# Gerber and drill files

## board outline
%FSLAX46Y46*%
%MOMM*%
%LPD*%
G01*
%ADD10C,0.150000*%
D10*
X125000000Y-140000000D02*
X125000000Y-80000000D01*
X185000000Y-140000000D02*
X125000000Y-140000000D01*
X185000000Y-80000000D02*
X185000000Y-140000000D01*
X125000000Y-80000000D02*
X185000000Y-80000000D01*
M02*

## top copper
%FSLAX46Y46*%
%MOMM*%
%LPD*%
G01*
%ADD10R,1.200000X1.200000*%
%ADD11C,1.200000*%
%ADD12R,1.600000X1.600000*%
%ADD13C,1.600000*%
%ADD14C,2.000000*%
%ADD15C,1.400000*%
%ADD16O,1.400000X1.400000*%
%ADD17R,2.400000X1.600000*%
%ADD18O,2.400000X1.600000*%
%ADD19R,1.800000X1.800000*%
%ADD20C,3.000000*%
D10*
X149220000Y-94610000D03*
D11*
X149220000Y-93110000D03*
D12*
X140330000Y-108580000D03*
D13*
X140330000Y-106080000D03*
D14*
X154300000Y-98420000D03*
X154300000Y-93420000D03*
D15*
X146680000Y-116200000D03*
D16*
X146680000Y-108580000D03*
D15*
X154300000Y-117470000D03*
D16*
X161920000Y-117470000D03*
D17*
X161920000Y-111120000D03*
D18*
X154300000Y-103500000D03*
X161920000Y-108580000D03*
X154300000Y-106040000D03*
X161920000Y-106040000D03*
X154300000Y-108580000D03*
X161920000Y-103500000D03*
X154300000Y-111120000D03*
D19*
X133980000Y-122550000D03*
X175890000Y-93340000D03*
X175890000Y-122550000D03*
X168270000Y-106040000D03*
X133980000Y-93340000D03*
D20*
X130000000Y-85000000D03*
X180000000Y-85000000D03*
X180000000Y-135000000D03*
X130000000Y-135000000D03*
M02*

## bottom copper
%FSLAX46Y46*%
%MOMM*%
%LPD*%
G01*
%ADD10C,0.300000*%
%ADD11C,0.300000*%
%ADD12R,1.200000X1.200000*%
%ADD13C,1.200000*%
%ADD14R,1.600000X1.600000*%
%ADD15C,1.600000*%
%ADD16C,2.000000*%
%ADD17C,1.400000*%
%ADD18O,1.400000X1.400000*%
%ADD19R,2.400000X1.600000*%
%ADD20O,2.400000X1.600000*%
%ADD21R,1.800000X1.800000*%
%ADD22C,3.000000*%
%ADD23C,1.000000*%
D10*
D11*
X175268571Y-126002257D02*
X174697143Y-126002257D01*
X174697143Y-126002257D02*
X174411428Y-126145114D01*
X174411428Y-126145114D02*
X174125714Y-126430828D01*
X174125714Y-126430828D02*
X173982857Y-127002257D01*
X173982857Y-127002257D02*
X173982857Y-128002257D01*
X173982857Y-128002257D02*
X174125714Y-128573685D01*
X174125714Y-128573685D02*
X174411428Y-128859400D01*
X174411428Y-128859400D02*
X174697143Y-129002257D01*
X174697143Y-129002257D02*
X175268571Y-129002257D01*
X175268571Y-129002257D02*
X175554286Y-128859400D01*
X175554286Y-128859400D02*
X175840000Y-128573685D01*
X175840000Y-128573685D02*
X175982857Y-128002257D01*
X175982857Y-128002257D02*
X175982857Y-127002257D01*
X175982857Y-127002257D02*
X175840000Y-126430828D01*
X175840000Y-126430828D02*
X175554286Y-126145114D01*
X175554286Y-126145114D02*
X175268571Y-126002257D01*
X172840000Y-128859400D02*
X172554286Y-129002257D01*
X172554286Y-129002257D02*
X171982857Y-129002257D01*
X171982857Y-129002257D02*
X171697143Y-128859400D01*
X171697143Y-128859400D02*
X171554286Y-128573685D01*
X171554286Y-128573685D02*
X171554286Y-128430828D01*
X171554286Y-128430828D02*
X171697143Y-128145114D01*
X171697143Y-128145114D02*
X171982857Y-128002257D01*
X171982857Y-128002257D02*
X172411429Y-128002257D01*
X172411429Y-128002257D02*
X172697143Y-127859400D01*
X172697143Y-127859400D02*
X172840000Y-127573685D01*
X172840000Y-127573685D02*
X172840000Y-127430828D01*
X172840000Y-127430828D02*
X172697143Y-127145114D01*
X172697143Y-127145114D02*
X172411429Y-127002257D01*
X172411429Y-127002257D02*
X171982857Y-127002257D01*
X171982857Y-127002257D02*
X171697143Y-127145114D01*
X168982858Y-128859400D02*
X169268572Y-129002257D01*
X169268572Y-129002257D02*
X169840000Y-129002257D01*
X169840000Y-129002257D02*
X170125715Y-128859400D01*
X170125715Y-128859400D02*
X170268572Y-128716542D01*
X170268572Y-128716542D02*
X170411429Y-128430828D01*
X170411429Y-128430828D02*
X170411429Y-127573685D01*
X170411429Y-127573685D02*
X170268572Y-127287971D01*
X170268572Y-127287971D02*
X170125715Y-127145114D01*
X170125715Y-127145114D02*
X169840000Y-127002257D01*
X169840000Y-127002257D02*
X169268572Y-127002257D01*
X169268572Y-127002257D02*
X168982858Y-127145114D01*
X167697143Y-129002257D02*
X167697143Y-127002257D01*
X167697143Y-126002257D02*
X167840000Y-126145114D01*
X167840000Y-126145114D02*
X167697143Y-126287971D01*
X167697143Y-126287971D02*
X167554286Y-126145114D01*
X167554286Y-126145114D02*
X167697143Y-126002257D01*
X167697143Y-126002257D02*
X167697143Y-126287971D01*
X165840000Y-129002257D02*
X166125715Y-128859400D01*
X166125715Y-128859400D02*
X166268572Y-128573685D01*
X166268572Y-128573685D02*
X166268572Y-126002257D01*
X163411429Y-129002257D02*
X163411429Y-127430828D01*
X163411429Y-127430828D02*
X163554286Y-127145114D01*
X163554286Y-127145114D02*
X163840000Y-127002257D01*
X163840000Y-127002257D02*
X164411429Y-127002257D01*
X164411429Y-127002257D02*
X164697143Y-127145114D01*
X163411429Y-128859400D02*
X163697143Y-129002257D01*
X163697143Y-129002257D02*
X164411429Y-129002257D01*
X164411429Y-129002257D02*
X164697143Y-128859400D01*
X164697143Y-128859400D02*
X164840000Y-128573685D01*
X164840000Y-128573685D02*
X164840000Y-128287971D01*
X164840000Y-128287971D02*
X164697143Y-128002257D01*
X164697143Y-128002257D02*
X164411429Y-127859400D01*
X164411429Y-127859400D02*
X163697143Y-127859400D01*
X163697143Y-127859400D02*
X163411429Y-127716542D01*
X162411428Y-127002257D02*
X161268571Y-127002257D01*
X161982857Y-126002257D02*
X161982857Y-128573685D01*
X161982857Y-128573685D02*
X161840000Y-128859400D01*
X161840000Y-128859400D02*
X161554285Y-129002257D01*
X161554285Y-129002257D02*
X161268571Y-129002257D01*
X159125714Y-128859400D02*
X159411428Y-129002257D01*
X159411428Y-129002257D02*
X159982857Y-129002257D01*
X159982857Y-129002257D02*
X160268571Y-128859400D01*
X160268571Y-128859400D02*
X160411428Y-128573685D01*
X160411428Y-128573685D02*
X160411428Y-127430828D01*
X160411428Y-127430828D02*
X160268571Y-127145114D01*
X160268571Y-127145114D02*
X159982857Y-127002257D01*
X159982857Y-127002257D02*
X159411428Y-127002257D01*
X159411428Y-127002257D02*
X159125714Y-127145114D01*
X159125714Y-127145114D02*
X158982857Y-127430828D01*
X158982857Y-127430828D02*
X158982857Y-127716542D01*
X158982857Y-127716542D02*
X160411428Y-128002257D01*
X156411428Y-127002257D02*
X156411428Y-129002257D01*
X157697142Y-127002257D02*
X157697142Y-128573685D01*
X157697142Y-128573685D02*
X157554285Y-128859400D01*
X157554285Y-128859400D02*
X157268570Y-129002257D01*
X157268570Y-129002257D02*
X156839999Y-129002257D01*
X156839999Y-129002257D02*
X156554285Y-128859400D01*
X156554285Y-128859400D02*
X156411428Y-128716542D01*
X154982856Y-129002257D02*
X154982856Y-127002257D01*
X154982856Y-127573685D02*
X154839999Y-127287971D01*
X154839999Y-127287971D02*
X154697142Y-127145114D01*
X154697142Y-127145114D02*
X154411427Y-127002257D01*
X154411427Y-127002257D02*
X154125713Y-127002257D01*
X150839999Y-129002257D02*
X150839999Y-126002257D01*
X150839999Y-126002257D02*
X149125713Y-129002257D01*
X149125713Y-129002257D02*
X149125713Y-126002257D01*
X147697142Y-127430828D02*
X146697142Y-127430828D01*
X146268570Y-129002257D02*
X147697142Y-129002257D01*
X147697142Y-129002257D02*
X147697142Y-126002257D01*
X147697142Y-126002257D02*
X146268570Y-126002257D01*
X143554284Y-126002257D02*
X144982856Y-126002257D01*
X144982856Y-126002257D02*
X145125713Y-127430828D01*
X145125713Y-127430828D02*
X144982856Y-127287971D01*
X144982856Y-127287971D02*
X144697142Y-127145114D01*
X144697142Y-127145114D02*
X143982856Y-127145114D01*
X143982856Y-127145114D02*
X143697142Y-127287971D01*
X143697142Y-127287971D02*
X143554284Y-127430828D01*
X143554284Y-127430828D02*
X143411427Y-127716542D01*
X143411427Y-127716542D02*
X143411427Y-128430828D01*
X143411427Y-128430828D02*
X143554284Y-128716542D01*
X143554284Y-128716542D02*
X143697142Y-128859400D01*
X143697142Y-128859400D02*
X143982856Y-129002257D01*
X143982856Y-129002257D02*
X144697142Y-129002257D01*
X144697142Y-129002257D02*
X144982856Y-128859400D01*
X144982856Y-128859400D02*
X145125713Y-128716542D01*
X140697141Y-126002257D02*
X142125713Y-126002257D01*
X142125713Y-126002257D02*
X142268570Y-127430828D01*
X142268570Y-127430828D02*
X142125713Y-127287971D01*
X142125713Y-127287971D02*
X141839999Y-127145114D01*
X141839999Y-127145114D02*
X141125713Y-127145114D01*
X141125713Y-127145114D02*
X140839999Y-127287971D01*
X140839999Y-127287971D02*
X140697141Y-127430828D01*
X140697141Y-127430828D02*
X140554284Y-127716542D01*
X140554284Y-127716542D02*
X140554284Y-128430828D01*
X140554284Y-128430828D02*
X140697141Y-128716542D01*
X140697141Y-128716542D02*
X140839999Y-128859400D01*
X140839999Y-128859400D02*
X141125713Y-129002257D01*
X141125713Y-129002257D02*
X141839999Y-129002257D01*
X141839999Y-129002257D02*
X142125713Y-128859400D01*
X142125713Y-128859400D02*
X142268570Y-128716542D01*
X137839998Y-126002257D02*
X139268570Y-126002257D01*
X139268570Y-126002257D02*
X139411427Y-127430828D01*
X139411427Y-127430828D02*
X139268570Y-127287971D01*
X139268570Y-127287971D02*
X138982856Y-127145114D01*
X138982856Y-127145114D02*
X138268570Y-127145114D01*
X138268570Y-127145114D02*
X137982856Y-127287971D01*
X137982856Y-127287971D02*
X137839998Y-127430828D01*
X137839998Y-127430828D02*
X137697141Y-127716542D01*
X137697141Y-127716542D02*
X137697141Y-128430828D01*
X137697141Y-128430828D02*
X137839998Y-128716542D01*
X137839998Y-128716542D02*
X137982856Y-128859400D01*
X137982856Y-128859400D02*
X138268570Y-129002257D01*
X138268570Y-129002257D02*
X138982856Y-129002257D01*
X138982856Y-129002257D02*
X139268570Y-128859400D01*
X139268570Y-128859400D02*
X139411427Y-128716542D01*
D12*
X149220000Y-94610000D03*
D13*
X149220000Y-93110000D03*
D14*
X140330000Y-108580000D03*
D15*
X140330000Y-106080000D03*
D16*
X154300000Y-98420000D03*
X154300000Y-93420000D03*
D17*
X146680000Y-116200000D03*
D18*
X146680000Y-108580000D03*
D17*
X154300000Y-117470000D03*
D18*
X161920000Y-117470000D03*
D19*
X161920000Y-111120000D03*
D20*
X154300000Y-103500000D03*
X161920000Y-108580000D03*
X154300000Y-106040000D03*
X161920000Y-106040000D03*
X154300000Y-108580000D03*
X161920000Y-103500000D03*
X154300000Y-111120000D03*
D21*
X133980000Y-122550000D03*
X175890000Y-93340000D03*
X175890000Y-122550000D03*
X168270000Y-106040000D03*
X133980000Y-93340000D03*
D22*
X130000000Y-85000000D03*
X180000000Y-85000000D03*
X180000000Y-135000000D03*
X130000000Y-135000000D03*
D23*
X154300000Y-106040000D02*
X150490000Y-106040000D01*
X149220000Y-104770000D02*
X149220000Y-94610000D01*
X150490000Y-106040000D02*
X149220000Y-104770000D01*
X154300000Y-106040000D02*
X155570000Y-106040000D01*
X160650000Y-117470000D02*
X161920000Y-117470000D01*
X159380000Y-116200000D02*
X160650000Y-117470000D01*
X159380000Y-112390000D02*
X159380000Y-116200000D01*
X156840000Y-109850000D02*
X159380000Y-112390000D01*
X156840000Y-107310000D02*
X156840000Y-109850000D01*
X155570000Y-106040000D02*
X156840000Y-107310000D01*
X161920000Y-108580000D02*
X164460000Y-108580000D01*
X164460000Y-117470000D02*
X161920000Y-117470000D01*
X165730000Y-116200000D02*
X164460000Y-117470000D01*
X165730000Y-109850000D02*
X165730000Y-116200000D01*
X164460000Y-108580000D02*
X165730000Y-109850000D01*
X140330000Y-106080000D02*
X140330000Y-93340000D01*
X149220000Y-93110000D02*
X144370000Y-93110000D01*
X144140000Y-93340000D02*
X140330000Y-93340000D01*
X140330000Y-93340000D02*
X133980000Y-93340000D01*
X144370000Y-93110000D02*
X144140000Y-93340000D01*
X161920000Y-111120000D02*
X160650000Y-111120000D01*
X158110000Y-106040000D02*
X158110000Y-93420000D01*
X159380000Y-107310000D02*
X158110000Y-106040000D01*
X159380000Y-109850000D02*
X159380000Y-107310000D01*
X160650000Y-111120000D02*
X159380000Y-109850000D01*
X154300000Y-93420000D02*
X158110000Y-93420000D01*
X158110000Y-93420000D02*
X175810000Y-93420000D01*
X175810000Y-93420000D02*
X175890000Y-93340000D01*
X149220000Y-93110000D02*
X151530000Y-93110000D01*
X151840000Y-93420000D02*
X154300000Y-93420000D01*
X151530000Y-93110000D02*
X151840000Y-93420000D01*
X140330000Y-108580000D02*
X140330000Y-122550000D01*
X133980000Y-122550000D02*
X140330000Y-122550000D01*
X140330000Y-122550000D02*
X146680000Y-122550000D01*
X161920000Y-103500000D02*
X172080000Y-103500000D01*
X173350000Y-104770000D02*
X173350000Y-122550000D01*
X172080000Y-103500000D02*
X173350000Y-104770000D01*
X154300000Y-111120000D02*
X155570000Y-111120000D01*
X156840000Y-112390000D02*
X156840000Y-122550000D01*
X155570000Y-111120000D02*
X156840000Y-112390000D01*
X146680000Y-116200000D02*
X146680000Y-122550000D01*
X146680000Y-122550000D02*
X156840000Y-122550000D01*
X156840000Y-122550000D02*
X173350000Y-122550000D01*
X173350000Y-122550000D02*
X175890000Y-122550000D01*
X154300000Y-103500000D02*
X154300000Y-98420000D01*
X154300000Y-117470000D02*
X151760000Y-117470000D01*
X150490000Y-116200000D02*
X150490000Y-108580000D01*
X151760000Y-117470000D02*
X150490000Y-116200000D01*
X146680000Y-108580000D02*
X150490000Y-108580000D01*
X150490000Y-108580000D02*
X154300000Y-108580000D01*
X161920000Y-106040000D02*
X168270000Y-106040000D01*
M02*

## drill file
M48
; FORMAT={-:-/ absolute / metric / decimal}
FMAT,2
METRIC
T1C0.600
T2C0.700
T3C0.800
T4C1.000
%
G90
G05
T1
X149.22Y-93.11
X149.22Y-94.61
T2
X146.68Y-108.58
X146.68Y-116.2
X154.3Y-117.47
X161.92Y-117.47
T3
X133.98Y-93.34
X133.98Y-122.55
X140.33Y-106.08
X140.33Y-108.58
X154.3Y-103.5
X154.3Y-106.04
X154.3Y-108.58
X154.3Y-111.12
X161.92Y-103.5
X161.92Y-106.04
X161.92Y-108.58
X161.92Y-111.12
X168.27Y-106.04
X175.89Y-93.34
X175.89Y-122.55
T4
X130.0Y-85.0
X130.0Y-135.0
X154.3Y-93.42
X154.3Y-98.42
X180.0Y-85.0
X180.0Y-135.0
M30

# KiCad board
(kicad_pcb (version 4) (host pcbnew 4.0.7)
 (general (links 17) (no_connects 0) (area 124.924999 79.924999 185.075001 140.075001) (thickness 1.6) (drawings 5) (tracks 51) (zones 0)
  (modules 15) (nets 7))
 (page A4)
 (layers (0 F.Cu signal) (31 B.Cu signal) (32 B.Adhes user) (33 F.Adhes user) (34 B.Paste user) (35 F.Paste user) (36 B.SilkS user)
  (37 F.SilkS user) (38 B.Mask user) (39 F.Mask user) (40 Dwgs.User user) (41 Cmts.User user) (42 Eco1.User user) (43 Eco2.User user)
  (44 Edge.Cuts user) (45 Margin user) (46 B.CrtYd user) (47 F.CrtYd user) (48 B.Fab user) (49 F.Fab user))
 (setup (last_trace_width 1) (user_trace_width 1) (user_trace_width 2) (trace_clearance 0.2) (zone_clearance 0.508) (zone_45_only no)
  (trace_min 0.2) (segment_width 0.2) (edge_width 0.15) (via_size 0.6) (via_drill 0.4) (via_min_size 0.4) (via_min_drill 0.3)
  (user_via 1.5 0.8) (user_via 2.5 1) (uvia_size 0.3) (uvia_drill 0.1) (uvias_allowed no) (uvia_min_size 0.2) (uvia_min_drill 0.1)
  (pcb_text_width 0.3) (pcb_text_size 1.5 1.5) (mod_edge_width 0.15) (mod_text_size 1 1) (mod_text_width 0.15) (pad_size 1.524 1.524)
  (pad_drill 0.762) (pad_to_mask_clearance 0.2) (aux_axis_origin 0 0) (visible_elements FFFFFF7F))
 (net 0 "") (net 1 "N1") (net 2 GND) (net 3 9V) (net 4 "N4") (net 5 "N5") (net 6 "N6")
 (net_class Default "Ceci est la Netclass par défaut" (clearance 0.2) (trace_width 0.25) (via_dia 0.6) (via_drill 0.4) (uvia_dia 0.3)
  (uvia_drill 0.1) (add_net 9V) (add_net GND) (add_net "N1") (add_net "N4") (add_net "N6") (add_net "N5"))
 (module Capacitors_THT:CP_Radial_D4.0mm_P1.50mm (layer F.Cu) (at 149.22 94.61 90)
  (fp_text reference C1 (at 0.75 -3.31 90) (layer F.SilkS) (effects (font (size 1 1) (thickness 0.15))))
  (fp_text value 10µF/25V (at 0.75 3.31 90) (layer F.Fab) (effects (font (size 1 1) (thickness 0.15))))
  (pad 1 thru_hole rect (at 0 0 90) (size 1.2 1.2) (drill 0.6) (layers *.Cu *.Mask) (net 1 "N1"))
  (pad 2 thru_hole circle (at 1.5 0 90) (size 1.2 1.2) (drill 0.6) (layers *.Cu *.Mask) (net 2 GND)))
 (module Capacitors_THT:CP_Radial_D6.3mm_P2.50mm (layer F.Cu) (at 140.33 108.58 90)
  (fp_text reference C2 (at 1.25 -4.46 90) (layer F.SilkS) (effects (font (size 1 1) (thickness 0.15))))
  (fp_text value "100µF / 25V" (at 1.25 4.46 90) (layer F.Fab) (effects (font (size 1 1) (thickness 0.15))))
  (pad 1 thru_hole rect (at 0 0 90) (size 1.6 1.6) (drill 0.8) (layers *.Cu *.Mask) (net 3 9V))
  (pad 2 thru_hole circle (at 2.5 0 90) (size 1.6 1.6) (drill 0.8) (layers *.Cu *.Mask) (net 2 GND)))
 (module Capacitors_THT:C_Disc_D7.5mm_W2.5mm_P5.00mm (layer F.Cu) (at 154.3 98.42 90)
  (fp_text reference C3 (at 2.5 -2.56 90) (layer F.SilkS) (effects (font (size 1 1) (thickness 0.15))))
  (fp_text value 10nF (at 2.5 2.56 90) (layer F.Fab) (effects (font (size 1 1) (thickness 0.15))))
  (pad 1 thru_hole circle (at 0 0 90) (size 2 2) (drill 1) (layers *.Cu *.Mask) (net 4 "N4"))
  (pad 2 thru_hole circle (at 5 0 90) (size 2 2) (drill 1) (layers *.Cu *.Mask) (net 2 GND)))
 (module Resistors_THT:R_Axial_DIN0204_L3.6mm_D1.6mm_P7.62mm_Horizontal (layer F.Cu) (at 146.68 116.2 90)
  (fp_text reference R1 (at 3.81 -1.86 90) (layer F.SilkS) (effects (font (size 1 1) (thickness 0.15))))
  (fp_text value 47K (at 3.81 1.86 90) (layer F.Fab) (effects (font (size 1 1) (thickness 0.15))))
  (pad 1 thru_hole circle (at 0 0 90) (size 1.4 1.4) (drill 0.7) (layers *.Cu *.Mask) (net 3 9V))
  (pad 2 thru_hole oval (at 7.62 0 90) (size 1.4 1.4) (drill 0.7) (layers *.Cu *.Mask) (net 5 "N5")))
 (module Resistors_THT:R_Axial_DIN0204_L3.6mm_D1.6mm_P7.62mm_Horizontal (layer F.Cu) (at 154.3 117.47)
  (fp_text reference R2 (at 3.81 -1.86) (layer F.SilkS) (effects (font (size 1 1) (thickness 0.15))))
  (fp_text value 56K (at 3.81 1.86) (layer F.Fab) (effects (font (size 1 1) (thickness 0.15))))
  (pad 1 thru_hole circle (at 0 0) (size 1.4 1.4) (drill 0.7) (layers *.Cu *.Mask) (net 5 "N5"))
  (pad 2 thru_hole oval (at 7.62 0) (size 1.4 1.4) (drill 0.7) (layers *.Cu *.Mask) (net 1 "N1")))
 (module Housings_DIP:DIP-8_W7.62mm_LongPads (layer F.Cu) (at 161.92 111.12 180)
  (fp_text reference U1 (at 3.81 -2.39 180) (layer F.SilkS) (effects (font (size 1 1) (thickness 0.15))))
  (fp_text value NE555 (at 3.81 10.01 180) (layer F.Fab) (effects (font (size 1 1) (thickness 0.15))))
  (pad 1 thru_hole rect (at 0 0 180) (size 2.4 1.6) (drill 0.8) (layers *.Cu *.Mask) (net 2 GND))
  (pad 5 thru_hole oval (at 7.62 7.62 180) (size 2.4 1.6) (drill 0.8) (layers *.Cu *.Mask) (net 4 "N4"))
  (pad 2 thru_hole oval (at 0 2.54 180) (size 2.4 1.6) (drill 0.8) (layers *.Cu *.Mask) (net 1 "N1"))
  (pad 6 thru_hole oval (at 7.62 5.08 180) (size 2.4 1.6) (drill 0.8) (layers *.Cu *.Mask) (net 1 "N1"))
  (pad 3 thru_hole oval (at 0 5.08 180) (size 2.4 1.6) (drill 0.8) (layers *.Cu *.Mask) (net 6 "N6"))
  (pad 7 thru_hole oval (at 7.62 2.54 180) (size 2.4 1.6) (drill 0.8) (layers *.Cu *.Mask) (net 5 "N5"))
  (pad 4 thru_hole oval (at 0 7.62 180) (size 2.4 1.6) (drill 0.8) (layers *.Cu *.Mask) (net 3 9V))
  (pad 8 thru_hole oval (at 7.62 0 180) (size 2.4 1.6) (drill 0.8) (layers *.Cu *.Mask) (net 3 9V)))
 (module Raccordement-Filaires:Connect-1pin (layer F.Cu) (at 133.98 122.55 90)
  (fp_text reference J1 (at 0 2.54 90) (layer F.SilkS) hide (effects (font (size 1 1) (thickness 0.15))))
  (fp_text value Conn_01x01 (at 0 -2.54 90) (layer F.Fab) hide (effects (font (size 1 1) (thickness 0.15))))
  (pad 1 thru_hole rect (at 0 0 90) (size 1.8 1.8) (drill 0.8) (layers *.Cu *.Mask) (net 3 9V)))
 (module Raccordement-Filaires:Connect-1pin (layer F.Cu) (at 175.89 93.34 270)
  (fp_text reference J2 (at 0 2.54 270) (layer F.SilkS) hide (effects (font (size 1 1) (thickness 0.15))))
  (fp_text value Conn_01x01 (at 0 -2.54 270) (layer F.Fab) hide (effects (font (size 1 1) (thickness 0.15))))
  (pad 1 thru_hole rect (at 0 0 270) (size 1.8 1.8) (drill 0.8) (layers *.Cu *.Mask) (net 2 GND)))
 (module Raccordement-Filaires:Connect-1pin (layer F.Cu) (at 175.89 122.55)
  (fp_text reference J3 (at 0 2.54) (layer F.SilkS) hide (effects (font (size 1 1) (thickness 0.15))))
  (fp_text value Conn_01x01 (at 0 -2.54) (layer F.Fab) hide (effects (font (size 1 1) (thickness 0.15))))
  (pad 1 thru_hole rect (at 0 0) (size 1.8 1.8) (drill 0.8) (layers *.Cu *.Mask) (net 3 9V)))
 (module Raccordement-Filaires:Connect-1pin (layer F.Cu) (at 168.27 106.04)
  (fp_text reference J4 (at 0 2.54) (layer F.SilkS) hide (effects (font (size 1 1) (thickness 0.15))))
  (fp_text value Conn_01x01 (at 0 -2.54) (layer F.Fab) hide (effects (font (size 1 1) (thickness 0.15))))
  (pad 1 thru_hole rect (at 0 0) (size 1.8 1.8) (drill 0.8) (layers *.Cu *.Mask) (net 6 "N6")))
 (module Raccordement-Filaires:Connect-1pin (layer F.Cu) (at 133.98 93.34)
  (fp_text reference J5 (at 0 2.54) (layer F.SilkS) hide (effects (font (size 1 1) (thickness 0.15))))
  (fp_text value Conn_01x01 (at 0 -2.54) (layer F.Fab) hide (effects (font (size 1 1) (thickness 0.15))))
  (pad 1 thru_hole rect (at 0 0) (size 1.8 1.8) (drill 0.8) (layers *.Cu *.Mask) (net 2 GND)))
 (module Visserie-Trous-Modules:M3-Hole (layer F.Cu) (at 130 85)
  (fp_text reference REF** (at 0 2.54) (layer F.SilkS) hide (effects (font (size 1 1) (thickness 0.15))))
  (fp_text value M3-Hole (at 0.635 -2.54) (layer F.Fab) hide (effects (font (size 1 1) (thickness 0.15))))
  (pad 1 thru_hole circle (at 0 0) (size 3 3) (drill 1) (layers *.Cu *.Mask)))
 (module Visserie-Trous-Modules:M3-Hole (layer F.Cu) (at 180 85)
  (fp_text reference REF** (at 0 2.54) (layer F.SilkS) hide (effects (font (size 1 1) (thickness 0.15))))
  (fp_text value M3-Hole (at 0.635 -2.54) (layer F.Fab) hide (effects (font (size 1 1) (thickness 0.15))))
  (pad 1 thru_hole circle (at 0 0) (size 3 3) (drill 1) (layers *.Cu *.Mask)))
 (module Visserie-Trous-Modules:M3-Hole (layer F.Cu) (at 180 135)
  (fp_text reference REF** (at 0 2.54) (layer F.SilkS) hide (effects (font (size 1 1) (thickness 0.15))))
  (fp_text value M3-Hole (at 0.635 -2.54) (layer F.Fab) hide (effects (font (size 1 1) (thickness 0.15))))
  (pad 1 thru_hole circle (at 0 0) (size 3 3) (drill 1) (layers *.Cu *.Mask)))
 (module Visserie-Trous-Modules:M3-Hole (layer F.Cu) (at 130 135)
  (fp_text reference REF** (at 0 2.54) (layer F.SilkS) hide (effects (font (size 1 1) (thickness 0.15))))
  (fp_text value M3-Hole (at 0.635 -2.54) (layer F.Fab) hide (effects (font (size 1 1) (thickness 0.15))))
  (pad 1 thru_hole circle (at 0 0) (size 3 3) (drill 1) (layers *.Cu *.Mask)))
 (gr_line (start 125 140) (end 125 80) (angle 90) (layer Edge.Cuts) (width 0.15))
 (gr_line (start 185 140) (end 125 140) (angle 90) (layer Edge.Cuts) (width 0.15))
 (gr_line (start 185 80) (end 185 140) (angle 90) (layer Edge.Cuts) (width 0.15))
 (gr_line (start 125 80) (end 185 80) (angle 90) (layer Edge.Cuts) (width 0.15))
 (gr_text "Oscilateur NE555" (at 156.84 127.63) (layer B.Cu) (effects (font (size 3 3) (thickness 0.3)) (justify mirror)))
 (segment (start 154.3 106.04) (end 150.49 106.04) (width 1) (layer B.Cu) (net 1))
 (segment (start 149.22 104.77) (end 149.22 94.61) (width 1) (layer B.Cu) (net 1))
 (segment (start 150.49 106.04) (end 149.22 104.77) (width 1) (layer B.Cu) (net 1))
 (segment (start 154.3 106.04) (end 155.57 106.04) (width 1) (layer B.Cu) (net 1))
 (segment (start 160.65 117.47) (end 161.92 117.47) (width 1) (layer B.Cu) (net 1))
 (segment (start 159.38 116.2) (end 160.65 117.47) (width 1) (layer B.Cu) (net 1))
 (segment (start 159.38 112.39) (end 159.38 116.2) (width 1) (layer B.Cu) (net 1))
 (segment (start 156.84 109.85) (end 159.38 112.39) (width 1) (layer B.Cu) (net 1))
 (segment (start 156.84 107.31) (end 156.84 109.85) (width 1) (layer B.Cu) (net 1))
 (segment (start 155.57 106.04) (end 156.84 107.31) (width 1) (layer B.Cu) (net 1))
 (segment (start 161.92 108.58) (end 164.46 108.58) (width 1) (layer B.Cu) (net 1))
 (segment (start 164.46 117.47) (end 161.92 117.47) (width 1) (layer B.Cu) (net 1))
 (segment (start 165.73 116.2) (end 164.46 117.47) (width 1) (layer B.Cu) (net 1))
 (segment (start 165.73 109.85) (end 165.73 116.2) (width 1) (layer B.Cu) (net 1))
 (segment (start 164.46 108.58) (end 165.73 109.85) (width 1) (layer B.Cu) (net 1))
 (segment (start 140.33 106.08) (end 140.33 93.34) (width 1) (layer B.Cu) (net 2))
 (segment (start 149.22 93.11) (end 144.37 93.11) (width 1) (layer B.Cu) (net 2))
 (segment (start 144.14 93.34) (end 140.33 93.34) (width 1) (layer B.Cu) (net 2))
 (segment (start 140.33 93.34) (end 133.98 93.34) (width 1) (layer B.Cu) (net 2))
 (segment (start 144.37 93.11) (end 144.14 93.34) (width 1) (layer B.Cu) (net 2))
 (segment (start 161.92 111.12) (end 160.65 111.12) (width 1) (layer B.Cu) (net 2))
 (segment (start 158.11 106.04) (end 158.11 93.42) (width 1) (layer B.Cu) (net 2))
 (segment (start 159.38 107.31) (end 158.11 106.04) (width 1) (layer B.Cu) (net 2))
 (segment (start 159.38 109.85) (end 159.38 107.31) (width 1) (layer B.Cu) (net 2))
 (segment (start 160.65 111.12) (end 159.38 109.85) (width 1) (layer B.Cu) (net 2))
 (segment (start 154.3 93.42) (end 158.11 93.42) (width 1) (layer B.Cu) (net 2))
 (segment (start 158.11 93.42) (end 175.81 93.42) (width 1) (layer B.Cu) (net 2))
 (segment (start 175.81 93.42) (end 175.89 93.34) (width 1) (layer B.Cu) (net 2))
 (segment (start 149.22 93.11) (end 151.53 93.11) (width 1) (layer B.Cu) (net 2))
 (segment (start 151.84 93.42) (end 154.3 93.42) (width 1) (layer B.Cu) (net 2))
 (segment (start 151.53 93.11) (end 151.84 93.42) (width 1) (layer B.Cu) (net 2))
 (segment (start 140.33 108.58) (end 140.33 122.55) (width 1) (layer B.Cu) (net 3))
 (segment (start 133.98 122.55) (end 140.33 122.55) (width 1) (layer B.Cu) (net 3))
 (segment (start 140.33 122.55) (end 146.68 122.55) (width 1) (layer B.Cu) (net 3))
 (segment (start 161.92 103.5) (end 172.08 103.5) (width 1) (layer B.Cu) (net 3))
 (segment (start 173.35 104.77) (end 173.35 122.55) (width 1) (layer B.Cu) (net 3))
 (segment (start 172.08 103.5) (end 173.35 104.77) (width 1) (layer B.Cu) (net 3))
 (segment (start 154.3 111.12) (end 155.57 111.12) (width 1) (layer B.Cu) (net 3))
 (segment (start 156.84 112.39) (end 156.84 122.55) (width 1) (layer B.Cu) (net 3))
 (segment (start 155.57 111.12) (end 156.84 112.39) (width 1) (layer B.Cu) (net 3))
 (segment (start 146.68 116.2) (end 146.68 122.55) (width 1) (layer B.Cu) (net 3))
 (segment (start 146.68 122.55) (end 156.84 122.55) (width 1) (layer B.Cu) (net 3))
 (segment (start 156.84 122.55) (end 173.35 122.55) (width 1) (layer B.Cu) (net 3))
 (segment (start 173.35 122.55) (end 175.89 122.55) (width 1) (layer B.Cu) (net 3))
 (segment (start 154.3 103.5) (end 154.3 98.42) (width 1) (layer B.Cu) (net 4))
 (segment (start 154.3 117.47) (end 151.76 117.47) (width 1) (layer B.Cu) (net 5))
 (segment (start 150.49 116.2) (end 150.49 108.58) (width 1) (layer B.Cu) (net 5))
 (segment (start 151.76 117.47) (end 150.49 116.2) (width 1) (layer B.Cu) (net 5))
 (segment (start 146.68 108.58) (end 150.49 108.58) (width 1) (layer B.Cu) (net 5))
 (segment (start 150.49 108.58) (end 154.3 108.58) (width 1) (layer B.Cu) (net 5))
 (segment (start 161.92 106.04) (end 168.27 106.04) (width 1) (layer B.Cu) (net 6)))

